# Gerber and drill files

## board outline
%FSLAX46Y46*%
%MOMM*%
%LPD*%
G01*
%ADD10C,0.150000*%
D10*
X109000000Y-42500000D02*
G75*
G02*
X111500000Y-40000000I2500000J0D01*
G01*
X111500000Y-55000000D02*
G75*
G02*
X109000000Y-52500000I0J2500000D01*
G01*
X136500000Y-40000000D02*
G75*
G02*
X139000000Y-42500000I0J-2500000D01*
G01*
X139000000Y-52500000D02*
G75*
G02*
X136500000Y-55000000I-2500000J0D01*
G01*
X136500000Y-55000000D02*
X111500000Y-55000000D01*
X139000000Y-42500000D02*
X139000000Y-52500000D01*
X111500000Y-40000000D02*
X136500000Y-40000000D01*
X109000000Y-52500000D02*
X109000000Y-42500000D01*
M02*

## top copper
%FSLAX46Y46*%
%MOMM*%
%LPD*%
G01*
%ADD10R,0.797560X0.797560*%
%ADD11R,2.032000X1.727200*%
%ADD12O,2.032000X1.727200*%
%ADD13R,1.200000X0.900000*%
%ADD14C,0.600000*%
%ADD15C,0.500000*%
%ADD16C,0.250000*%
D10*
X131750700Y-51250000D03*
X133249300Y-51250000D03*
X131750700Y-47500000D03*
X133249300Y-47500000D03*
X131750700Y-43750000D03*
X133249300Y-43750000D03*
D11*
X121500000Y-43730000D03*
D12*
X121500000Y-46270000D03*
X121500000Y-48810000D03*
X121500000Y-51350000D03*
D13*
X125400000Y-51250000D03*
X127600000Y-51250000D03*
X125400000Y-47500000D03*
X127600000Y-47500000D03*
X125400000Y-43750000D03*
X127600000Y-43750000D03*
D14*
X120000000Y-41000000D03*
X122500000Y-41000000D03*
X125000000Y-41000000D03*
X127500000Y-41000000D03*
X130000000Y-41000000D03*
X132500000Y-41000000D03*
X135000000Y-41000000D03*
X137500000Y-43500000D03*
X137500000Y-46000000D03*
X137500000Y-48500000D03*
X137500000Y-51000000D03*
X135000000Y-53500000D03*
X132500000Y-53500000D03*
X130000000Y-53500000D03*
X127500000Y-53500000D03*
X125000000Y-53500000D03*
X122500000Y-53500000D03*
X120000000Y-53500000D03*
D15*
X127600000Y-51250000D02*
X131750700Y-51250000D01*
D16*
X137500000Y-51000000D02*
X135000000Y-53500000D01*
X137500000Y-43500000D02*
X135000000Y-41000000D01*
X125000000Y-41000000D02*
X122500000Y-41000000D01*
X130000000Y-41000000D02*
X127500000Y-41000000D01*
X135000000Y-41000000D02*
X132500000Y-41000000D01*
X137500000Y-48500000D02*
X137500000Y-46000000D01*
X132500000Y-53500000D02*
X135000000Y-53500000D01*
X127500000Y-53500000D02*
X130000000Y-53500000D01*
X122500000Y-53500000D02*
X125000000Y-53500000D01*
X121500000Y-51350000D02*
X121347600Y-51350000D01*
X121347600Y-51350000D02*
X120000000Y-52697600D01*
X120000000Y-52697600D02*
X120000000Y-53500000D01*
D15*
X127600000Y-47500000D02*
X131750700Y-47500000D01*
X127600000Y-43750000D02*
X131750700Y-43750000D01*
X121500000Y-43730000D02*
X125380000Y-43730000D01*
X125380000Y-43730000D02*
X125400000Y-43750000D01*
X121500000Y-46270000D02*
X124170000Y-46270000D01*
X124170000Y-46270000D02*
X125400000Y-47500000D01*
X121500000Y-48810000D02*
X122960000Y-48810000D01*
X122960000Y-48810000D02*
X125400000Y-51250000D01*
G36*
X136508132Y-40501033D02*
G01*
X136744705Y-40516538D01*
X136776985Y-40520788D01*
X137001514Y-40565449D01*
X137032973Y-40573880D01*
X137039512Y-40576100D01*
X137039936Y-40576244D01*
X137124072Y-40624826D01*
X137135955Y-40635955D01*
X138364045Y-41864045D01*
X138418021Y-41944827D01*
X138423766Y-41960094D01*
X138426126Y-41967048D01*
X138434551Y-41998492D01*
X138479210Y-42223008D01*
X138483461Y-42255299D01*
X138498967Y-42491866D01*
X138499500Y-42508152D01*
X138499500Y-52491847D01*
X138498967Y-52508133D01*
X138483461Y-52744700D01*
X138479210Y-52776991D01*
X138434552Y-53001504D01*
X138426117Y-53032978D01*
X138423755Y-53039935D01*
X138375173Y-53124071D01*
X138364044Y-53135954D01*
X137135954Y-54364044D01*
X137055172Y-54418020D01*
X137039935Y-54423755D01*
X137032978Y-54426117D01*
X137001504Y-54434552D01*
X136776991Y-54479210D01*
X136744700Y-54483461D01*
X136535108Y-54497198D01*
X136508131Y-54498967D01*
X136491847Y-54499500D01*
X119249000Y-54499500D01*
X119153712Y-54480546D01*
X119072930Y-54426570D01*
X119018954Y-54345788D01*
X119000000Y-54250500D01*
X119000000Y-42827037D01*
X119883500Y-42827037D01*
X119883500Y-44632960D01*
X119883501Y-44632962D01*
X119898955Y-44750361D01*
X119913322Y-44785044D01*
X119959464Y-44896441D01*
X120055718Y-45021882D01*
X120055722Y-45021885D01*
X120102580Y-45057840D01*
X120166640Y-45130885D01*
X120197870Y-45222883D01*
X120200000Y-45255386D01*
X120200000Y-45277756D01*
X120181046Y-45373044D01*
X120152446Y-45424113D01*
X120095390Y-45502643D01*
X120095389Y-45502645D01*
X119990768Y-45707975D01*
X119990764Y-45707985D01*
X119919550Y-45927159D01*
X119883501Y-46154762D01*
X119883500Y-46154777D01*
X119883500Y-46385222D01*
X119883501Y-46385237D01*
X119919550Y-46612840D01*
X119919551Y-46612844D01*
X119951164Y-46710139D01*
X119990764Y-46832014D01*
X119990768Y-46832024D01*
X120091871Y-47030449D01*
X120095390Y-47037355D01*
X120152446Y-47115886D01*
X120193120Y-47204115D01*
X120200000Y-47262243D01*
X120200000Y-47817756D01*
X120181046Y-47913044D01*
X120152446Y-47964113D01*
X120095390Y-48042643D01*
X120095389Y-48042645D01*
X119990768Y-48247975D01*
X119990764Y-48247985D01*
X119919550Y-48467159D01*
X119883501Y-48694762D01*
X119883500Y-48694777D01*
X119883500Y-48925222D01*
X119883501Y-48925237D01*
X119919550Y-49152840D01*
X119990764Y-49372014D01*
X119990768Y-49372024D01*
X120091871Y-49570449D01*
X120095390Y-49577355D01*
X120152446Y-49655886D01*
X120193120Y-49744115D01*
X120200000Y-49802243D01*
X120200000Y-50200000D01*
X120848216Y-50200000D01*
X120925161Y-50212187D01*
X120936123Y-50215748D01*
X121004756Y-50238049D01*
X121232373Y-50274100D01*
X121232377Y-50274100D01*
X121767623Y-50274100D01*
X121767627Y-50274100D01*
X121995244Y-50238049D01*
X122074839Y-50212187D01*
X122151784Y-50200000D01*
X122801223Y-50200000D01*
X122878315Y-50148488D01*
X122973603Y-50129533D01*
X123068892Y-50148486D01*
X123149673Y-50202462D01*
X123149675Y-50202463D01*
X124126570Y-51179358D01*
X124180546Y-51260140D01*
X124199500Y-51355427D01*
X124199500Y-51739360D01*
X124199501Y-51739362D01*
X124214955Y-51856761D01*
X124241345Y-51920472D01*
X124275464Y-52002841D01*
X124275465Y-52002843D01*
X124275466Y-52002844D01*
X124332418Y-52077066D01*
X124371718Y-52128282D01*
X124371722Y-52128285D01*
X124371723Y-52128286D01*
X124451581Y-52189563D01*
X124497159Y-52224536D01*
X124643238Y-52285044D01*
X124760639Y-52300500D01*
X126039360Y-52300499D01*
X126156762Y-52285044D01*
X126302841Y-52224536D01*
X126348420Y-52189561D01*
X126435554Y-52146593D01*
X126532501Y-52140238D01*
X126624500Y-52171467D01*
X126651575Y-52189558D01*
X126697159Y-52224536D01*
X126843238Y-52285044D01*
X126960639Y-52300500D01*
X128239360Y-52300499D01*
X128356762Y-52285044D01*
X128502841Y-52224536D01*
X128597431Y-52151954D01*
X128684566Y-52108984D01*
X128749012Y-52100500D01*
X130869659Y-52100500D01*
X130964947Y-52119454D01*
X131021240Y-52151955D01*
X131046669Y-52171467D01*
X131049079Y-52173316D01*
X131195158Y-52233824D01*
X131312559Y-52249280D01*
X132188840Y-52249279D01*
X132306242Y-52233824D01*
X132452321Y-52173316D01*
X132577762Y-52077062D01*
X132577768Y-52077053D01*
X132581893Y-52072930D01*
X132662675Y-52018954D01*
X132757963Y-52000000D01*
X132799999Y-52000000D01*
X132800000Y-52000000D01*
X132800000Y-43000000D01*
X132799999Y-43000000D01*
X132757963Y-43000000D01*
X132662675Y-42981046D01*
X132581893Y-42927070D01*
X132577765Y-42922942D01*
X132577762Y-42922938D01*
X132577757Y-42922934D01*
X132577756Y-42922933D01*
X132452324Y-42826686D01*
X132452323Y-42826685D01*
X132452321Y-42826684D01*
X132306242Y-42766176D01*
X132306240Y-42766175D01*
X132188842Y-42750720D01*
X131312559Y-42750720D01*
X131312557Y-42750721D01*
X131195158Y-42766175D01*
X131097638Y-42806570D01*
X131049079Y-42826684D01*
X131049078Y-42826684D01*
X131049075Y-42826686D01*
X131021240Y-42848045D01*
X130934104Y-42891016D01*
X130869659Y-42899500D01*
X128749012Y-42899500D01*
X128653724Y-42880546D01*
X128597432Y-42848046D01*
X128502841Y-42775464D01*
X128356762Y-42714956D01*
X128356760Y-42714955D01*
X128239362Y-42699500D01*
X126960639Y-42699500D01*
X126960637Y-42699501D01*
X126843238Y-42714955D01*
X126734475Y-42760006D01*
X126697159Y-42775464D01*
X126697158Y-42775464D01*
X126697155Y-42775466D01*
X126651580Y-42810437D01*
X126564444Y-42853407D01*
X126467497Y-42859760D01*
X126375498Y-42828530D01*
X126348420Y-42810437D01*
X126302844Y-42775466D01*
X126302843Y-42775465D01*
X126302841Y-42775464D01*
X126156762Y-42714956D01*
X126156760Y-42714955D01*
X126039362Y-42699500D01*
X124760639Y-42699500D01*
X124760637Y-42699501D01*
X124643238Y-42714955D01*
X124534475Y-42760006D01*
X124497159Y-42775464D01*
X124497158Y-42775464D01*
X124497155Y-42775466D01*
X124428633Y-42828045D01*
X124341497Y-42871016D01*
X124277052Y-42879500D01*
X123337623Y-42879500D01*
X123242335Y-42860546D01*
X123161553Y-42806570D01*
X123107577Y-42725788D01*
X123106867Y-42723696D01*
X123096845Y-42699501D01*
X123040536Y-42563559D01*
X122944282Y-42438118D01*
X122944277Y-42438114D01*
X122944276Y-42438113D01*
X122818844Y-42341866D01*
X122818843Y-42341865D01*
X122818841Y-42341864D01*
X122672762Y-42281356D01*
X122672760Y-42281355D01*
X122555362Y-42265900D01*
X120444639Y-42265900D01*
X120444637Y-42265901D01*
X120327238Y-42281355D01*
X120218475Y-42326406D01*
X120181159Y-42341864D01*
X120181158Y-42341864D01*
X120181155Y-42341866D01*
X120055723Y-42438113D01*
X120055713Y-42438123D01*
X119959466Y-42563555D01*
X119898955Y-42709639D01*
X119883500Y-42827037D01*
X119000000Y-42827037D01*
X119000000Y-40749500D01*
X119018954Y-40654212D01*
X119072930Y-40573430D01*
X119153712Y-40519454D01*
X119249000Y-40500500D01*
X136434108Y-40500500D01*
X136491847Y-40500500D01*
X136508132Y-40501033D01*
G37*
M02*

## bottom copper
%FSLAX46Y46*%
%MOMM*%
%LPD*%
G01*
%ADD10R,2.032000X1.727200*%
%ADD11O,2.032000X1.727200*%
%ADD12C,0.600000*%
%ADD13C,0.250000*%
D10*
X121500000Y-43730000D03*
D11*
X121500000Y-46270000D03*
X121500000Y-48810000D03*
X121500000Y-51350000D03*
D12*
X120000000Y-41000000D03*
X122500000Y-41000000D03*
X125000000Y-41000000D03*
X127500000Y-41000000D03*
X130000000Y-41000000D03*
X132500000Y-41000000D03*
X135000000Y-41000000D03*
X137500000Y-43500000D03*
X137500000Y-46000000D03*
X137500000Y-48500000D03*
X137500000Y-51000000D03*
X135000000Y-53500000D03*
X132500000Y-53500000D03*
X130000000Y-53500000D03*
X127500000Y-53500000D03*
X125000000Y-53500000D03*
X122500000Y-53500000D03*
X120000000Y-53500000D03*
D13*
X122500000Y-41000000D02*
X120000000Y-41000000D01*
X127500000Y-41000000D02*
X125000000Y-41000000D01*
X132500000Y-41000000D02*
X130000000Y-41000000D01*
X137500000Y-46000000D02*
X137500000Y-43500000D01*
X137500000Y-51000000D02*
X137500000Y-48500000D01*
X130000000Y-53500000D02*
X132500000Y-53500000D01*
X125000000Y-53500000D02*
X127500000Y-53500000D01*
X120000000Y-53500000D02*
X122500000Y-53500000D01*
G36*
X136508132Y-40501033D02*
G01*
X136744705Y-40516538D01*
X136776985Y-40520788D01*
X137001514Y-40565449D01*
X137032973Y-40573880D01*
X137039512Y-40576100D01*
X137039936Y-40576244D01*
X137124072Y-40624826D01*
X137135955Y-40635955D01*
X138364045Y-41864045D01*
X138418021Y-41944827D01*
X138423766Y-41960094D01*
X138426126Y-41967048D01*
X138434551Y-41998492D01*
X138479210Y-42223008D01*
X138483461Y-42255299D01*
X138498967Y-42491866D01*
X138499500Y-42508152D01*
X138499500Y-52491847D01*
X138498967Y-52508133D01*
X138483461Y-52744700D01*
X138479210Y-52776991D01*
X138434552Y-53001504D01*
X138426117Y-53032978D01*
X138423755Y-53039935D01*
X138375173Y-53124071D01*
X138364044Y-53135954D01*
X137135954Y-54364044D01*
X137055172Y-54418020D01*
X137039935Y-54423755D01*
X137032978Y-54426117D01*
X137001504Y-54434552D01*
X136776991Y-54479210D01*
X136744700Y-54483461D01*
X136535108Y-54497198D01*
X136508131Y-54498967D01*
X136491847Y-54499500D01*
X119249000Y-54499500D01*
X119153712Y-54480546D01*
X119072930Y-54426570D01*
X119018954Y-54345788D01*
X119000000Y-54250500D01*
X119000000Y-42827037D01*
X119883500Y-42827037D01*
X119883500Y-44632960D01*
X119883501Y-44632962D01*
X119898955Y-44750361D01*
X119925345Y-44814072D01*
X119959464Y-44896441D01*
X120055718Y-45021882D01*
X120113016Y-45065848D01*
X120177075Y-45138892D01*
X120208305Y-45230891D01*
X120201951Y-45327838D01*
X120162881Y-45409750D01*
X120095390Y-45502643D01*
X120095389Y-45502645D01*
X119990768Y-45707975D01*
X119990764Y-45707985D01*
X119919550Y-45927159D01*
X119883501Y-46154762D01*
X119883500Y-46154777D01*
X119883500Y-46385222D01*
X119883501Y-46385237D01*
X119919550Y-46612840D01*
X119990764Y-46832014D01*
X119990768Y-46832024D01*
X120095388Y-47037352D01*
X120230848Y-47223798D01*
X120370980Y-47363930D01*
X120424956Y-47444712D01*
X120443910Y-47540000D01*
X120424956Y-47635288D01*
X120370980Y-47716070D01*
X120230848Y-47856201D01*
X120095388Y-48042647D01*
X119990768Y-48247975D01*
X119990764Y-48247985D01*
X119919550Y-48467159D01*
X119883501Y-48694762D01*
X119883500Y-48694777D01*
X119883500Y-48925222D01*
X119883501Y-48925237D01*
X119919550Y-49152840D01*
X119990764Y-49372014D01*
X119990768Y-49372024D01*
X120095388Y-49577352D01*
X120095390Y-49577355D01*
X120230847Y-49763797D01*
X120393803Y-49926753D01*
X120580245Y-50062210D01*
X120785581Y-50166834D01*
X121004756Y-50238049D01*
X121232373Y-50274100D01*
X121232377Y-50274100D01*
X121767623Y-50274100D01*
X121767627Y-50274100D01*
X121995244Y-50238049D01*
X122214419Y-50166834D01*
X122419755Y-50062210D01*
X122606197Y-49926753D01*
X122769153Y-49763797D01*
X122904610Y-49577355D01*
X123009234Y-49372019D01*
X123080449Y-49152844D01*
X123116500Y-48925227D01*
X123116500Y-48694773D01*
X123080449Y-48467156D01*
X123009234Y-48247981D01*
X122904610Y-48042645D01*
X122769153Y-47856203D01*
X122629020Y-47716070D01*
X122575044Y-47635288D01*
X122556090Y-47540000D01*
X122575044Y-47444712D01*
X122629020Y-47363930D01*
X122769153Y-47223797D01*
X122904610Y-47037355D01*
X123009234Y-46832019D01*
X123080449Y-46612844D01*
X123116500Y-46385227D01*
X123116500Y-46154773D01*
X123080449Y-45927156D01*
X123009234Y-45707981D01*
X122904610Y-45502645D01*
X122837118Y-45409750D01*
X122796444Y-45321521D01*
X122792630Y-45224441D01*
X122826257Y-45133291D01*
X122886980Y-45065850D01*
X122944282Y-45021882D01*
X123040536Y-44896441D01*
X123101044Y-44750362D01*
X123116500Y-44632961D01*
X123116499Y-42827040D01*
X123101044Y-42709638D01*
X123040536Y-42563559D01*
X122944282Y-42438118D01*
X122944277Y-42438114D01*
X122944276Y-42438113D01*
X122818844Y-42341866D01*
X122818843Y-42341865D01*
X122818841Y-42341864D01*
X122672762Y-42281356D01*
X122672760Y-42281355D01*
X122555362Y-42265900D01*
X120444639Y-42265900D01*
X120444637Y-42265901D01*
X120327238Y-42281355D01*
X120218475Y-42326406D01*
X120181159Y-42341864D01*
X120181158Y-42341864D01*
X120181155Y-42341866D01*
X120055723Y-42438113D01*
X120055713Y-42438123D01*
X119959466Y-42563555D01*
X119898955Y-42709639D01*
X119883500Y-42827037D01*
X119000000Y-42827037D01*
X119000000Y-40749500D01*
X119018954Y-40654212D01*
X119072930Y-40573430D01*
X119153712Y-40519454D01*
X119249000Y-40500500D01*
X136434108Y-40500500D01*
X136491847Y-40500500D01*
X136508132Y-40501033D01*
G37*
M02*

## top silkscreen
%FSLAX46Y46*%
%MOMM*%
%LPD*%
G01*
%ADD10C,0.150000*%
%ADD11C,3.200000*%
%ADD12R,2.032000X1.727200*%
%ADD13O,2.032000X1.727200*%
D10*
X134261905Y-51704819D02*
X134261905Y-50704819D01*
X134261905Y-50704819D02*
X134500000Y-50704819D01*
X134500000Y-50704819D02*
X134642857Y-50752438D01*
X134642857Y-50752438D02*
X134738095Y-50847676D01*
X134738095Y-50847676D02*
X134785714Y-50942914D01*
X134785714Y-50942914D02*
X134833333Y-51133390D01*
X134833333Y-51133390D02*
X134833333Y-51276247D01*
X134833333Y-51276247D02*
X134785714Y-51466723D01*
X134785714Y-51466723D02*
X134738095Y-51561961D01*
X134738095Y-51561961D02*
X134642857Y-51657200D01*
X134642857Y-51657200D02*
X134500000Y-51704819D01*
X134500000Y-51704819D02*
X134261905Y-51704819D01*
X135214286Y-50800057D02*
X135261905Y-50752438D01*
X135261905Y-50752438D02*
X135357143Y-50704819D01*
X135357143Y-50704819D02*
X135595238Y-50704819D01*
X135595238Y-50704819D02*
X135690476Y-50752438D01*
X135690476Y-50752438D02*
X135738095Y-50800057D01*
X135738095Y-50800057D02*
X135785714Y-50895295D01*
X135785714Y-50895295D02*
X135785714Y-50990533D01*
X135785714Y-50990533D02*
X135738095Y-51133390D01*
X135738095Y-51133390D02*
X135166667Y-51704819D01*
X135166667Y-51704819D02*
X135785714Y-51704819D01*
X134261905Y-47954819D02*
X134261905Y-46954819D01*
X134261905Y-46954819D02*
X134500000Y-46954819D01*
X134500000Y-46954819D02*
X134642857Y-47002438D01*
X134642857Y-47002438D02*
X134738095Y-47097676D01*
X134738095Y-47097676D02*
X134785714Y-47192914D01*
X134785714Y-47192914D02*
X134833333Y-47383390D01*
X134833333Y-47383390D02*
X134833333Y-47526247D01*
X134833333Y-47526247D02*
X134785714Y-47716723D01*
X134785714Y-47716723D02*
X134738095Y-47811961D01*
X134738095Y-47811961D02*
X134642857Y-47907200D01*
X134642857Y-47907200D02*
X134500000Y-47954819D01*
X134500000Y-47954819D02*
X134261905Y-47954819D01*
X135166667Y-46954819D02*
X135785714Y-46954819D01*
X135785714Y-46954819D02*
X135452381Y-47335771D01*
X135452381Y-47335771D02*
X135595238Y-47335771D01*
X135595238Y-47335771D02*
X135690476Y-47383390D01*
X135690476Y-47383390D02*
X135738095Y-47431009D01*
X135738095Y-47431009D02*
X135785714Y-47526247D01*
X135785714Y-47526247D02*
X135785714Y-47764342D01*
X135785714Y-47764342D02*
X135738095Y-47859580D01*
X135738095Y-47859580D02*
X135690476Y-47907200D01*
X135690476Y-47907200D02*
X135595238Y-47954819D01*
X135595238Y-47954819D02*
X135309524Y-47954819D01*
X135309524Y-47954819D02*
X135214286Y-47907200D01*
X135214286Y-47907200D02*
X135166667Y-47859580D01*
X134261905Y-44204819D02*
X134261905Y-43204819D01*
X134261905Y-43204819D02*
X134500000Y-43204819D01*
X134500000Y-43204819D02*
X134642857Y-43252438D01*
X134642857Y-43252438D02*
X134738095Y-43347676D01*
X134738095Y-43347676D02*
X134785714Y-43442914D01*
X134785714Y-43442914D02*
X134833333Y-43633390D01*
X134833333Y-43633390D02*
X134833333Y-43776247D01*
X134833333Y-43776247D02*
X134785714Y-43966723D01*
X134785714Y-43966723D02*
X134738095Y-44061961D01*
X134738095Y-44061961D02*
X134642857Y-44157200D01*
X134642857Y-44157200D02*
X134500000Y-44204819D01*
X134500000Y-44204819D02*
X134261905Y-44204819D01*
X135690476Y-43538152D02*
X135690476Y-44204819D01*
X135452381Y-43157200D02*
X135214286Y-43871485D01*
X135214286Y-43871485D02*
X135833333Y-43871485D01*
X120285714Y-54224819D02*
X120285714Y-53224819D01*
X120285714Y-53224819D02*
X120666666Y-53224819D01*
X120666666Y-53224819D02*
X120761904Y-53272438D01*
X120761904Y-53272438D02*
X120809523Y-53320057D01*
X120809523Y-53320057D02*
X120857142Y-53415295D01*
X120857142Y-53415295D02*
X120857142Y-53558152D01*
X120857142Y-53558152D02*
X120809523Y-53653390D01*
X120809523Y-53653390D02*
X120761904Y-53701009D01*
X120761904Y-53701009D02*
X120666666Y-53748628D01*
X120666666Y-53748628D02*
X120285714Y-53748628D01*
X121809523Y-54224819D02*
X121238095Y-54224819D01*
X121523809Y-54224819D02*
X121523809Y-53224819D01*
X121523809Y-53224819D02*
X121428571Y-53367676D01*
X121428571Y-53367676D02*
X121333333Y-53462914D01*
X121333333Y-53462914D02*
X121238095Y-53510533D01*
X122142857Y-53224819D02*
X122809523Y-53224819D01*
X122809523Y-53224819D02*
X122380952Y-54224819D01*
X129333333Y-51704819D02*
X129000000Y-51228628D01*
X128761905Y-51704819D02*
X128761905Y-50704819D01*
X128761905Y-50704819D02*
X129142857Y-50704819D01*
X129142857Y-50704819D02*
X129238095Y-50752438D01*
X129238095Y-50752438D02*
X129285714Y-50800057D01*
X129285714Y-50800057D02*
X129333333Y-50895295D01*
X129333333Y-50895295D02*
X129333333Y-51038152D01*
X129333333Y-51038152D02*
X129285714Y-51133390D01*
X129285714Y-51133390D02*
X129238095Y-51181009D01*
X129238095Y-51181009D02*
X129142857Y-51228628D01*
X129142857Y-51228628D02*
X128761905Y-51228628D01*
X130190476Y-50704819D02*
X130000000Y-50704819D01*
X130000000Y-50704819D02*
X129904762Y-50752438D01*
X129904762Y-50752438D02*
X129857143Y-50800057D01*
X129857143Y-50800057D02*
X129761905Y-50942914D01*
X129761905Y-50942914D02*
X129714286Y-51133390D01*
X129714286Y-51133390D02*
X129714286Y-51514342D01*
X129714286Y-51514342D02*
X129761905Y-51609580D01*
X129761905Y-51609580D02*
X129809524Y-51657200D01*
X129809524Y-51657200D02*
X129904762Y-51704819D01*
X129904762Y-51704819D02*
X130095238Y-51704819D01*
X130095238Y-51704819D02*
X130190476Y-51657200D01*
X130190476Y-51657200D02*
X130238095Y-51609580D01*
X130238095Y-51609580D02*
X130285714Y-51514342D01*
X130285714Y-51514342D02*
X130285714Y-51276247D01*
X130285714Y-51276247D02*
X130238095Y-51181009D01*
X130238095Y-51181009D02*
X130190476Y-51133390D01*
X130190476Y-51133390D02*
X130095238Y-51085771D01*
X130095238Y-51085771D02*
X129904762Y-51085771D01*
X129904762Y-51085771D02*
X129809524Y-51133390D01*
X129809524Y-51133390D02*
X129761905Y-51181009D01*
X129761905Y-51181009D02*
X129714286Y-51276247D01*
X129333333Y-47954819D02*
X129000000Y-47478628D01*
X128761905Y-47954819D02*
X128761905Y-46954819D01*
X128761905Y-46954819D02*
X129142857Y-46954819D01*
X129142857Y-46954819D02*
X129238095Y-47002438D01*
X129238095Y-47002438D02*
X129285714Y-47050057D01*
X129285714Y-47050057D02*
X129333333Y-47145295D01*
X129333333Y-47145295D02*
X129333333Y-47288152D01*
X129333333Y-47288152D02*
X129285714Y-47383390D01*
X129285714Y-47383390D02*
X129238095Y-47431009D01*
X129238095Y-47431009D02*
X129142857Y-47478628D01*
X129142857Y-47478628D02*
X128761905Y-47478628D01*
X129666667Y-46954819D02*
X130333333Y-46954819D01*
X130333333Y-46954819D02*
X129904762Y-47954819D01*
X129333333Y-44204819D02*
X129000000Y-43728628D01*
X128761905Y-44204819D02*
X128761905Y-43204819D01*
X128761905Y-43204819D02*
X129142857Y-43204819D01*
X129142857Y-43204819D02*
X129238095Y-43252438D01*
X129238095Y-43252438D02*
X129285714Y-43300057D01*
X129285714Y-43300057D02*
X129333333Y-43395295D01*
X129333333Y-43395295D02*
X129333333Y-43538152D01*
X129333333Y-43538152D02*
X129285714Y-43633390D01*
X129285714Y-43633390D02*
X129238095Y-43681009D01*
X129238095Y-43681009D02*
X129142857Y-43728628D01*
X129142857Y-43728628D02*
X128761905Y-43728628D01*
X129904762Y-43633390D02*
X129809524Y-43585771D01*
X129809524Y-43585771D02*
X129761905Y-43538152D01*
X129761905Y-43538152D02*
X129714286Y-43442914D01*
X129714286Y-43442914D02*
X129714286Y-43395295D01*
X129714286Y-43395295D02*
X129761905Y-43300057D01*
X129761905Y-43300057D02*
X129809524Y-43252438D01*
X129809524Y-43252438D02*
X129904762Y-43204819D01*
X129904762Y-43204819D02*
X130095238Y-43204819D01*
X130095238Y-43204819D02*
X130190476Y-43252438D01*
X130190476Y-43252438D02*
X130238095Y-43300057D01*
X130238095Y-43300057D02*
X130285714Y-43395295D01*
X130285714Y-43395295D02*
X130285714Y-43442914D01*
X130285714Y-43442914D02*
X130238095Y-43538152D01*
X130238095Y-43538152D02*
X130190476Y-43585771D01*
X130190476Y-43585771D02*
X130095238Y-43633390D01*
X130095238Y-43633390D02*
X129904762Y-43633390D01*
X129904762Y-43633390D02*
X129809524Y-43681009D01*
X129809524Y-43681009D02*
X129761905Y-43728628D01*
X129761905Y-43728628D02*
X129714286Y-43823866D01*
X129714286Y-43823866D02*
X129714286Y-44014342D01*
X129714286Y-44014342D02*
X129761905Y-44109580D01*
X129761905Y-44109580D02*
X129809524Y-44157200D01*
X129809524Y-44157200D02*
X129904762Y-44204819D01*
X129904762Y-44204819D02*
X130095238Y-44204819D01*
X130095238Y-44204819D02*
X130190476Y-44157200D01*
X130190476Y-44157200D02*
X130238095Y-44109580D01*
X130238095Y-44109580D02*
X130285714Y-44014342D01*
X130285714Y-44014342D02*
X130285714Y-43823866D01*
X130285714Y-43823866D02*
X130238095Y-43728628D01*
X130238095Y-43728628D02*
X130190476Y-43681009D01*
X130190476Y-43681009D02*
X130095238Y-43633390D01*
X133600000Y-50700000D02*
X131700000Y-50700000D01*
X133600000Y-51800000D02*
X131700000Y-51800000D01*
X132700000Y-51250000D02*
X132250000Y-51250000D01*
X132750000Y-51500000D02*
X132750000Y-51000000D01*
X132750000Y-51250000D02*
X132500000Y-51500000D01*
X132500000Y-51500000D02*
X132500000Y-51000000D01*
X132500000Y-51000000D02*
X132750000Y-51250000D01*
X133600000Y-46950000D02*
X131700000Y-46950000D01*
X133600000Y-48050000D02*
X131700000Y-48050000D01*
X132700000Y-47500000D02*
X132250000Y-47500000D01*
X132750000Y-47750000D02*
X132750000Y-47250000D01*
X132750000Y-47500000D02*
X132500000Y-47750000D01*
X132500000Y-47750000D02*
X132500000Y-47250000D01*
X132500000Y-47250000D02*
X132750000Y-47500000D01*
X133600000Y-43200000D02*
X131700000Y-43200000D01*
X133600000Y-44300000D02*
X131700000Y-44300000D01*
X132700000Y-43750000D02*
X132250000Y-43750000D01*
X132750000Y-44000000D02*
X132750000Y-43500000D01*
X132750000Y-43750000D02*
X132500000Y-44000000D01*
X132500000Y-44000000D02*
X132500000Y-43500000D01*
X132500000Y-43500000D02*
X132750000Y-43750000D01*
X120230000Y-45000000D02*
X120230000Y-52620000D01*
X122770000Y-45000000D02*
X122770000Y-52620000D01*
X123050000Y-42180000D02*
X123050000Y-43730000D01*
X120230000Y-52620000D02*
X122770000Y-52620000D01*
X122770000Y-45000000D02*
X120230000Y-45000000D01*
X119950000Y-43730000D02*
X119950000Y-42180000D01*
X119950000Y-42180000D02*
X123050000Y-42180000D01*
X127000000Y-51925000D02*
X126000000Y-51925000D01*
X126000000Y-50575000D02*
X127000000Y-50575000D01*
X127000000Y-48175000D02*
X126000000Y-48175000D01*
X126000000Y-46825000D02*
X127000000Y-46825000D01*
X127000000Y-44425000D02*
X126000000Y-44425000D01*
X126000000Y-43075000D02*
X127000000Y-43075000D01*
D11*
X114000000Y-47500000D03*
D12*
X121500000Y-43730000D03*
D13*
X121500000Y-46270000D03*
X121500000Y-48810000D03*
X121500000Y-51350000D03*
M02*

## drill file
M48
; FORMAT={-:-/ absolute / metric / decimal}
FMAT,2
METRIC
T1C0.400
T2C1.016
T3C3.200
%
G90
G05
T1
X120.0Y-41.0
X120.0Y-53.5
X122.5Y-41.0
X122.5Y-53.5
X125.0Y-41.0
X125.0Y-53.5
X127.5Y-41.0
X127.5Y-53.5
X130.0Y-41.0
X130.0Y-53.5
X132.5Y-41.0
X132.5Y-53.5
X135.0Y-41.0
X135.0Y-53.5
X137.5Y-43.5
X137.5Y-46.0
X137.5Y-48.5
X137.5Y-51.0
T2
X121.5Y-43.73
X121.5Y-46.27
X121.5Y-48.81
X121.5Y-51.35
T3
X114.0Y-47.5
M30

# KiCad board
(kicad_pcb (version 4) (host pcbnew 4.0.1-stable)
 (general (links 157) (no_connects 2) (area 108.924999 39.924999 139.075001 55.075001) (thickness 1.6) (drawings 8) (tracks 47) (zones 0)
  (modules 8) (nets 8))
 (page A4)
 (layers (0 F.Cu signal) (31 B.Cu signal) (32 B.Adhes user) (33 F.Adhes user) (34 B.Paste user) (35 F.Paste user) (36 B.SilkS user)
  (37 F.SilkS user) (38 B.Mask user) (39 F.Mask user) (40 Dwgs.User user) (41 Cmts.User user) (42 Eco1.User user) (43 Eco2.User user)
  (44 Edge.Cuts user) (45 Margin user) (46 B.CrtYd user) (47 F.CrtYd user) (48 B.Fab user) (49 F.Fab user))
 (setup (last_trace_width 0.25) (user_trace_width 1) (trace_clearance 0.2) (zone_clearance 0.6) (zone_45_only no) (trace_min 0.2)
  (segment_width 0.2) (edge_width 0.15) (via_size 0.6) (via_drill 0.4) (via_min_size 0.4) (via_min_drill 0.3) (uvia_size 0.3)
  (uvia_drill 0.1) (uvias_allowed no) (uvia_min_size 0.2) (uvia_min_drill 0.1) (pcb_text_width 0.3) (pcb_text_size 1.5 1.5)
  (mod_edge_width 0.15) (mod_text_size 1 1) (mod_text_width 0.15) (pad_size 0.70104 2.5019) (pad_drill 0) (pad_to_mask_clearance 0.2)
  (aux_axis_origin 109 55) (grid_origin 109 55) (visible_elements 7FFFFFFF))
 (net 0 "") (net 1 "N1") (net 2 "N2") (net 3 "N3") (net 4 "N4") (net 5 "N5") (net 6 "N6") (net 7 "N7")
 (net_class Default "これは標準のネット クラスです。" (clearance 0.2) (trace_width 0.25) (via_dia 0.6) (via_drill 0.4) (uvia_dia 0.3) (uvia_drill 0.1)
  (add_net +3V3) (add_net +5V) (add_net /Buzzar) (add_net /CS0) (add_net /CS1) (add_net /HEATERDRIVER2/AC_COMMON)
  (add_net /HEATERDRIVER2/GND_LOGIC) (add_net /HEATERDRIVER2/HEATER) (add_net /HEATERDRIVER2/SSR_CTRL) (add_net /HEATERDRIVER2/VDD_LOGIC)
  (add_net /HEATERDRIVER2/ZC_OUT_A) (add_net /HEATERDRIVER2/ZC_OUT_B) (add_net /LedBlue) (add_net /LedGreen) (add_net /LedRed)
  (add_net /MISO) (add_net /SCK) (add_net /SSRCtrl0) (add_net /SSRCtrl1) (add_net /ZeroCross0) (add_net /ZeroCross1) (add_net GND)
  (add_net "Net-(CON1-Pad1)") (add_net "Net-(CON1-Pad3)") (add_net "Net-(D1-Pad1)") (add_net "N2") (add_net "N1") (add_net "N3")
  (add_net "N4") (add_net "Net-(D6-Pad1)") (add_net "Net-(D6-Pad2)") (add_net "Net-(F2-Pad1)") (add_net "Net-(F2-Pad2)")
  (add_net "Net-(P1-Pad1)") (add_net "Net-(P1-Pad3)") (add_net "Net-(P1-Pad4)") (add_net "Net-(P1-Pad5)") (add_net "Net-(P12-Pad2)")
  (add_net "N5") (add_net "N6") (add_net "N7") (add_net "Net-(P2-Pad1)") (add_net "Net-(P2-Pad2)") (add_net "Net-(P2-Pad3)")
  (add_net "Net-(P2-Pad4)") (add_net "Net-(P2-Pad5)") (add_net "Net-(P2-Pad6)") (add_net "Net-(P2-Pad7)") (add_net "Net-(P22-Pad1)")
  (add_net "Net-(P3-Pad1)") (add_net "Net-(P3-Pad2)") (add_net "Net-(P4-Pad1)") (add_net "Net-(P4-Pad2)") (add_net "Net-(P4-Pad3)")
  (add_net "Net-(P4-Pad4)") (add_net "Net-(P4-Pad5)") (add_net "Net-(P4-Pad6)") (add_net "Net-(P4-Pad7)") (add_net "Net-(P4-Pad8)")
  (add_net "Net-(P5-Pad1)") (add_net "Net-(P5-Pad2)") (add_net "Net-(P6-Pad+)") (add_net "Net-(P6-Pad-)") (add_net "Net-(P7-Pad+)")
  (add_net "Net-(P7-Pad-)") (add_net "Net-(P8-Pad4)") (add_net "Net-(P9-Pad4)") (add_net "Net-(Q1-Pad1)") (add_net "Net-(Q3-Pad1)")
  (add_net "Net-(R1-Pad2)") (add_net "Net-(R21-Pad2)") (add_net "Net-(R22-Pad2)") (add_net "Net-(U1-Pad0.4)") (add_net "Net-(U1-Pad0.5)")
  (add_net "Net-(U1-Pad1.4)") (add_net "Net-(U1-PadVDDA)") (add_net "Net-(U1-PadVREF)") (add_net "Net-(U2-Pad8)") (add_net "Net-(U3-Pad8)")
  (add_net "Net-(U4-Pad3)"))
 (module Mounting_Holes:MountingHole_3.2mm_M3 (layer F.Cu) (at 114 47.5 90)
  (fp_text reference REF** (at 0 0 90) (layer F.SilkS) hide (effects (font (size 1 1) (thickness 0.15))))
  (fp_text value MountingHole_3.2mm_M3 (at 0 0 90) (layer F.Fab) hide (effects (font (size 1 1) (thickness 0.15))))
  (pad 1 np_thru_hole circle (at 0 0 90) (size 3.2 3.2) (drill 3.2) (layers *.Cu *.Mask F.SilkS)))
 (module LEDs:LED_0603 (layer F.Cu) (at 132.5 51.25 180)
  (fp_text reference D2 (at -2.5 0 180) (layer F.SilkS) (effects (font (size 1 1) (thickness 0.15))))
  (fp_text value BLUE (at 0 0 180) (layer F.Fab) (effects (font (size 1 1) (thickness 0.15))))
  (fp_line (start -1.1 0.55) (end 0.8 0.55) (layer F.SilkS) (width 0.15))
  (fp_line (start -1.1 -0.55) (end 0.8 -0.55) (layer F.SilkS) (width 0.15))
  (fp_line (start -0.2 0) (end 0.25 0) (layer F.SilkS) (width 0.15))
  (fp_line (start -0.25 -0.25) (end -0.25 0.25) (layer F.SilkS) (width 0.15))
  (fp_line (start -0.25 0) (end 0 -0.25) (layer F.SilkS) (width 0.15))
  (fp_line (start 0 -0.25) (end 0 0.25) (layer F.SilkS) (width 0.15))
  (fp_line (start 0 0.25) (end -0.25 0) (layer F.SilkS) (width 0.15))
  (pad 2 smd rect (at 0.7493 0) (size 0.79756 0.79756) (layers F.Cu F.Paste F.Mask) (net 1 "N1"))
  (pad 1 smd rect (at -0.7493 0) (size 0.79756 0.79756) (layers F.Cu F.Paste F.Mask) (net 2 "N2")))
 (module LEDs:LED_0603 (layer F.Cu) (at 132.5 47.5 180)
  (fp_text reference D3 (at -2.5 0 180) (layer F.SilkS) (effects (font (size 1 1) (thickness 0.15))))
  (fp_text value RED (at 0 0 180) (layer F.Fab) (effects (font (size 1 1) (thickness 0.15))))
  (fp_line (start -1.1 0.55) (end 0.8 0.55) (layer F.SilkS) (width 0.15))
  (fp_line (start -1.1 -0.55) (end 0.8 -0.55) (layer F.SilkS) (width 0.15))
  (fp_line (start -0.2 0) (end 0.25 0) (layer F.SilkS) (width 0.15))
  (fp_line (start -0.25 -0.25) (end -0.25 0.25) (layer F.SilkS) (width 0.15))
  (fp_line (start -0.25 0) (end 0 -0.25) (layer F.SilkS) (width 0.15))
  (fp_line (start 0 -0.25) (end 0 0.25) (layer F.SilkS) (width 0.15))
  (fp_line (start 0 0.25) (end -0.25 0) (layer F.SilkS) (width 0.15))
  (pad 2 smd rect (at 0.7493 0) (size 0.79756 0.79756) (layers F.Cu F.Paste F.Mask) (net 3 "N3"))
  (pad 1 smd rect (at -0.7493 0) (size 0.79756 0.79756) (layers F.Cu F.Paste F.Mask) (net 2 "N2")))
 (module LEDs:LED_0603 (layer F.Cu) (at 132.5 43.75 180)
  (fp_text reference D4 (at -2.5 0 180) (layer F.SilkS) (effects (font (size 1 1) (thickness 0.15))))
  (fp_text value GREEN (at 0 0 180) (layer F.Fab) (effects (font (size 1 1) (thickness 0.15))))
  (fp_line (start -1.1 0.55) (end 0.8 0.55) (layer F.SilkS) (width 0.15))
  (fp_line (start -1.1 -0.55) (end 0.8 -0.55) (layer F.SilkS) (width 0.15))
  (fp_line (start -0.2 0) (end 0.25 0) (layer F.SilkS) (width 0.15))
  (fp_line (start -0.25 -0.25) (end -0.25 0.25) (layer F.SilkS) (width 0.15))
  (fp_line (start -0.25 0) (end 0 -0.25) (layer F.SilkS) (width 0.15))
  (fp_line (start 0 -0.25) (end 0 0.25) (layer F.SilkS) (width 0.15))
  (fp_line (start 0 0.25) (end -0.25 0) (layer F.SilkS) (width 0.15))
  (pad 2 smd rect (at 0.7493 0) (size 0.79756 0.79756) (layers F.Cu F.Paste F.Mask) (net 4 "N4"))
  (pad 1 smd rect (at -0.7493 0) (size 0.79756 0.79756) (layers F.Cu F.Paste F.Mask) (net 2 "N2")))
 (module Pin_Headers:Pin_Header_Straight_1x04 (layer F.Cu) (at 121.5 43.73)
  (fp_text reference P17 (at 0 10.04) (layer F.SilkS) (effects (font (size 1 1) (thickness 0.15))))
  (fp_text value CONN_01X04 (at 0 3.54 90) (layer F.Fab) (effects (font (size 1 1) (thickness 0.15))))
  (fp_line (start -1.27 1.27) (end -1.27 8.89) (layer F.SilkS) (width 0.15))
  (fp_line (start 1.27 1.27) (end 1.27 8.89) (layer F.SilkS) (width 0.15))
  (fp_line (start 1.55 -1.55) (end 1.55 0) (layer F.SilkS) (width 0.15))
  (fp_line (start -1.27 8.89) (end 1.27 8.89) (layer F.SilkS) (width 0.15))
  (fp_line (start 1.27 1.27) (end -1.27 1.27) (layer F.SilkS) (width 0.15))
  (fp_line (start -1.55 0) (end -1.55 -1.55) (layer F.SilkS) (width 0.15))
  (fp_line (start -1.55 -1.55) (end 1.55 -1.55) (layer F.SilkS) (width 0.15))
  (pad 1 thru_hole rect (at 0 0) (size 2.032 1.7272) (drill 1.016) (layers *.Cu *.Mask F.SilkS) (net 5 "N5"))
  (pad 2 thru_hole oval (at 0 2.54) (size 2.032 1.7272) (drill 1.016) (layers *.Cu *.Mask F.SilkS) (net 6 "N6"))
  (pad 3 thru_hole oval (at 0 5.08) (size 2.032 1.7272) (drill 1.016) (layers *.Cu *.Mask F.SilkS) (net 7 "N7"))
  (pad 4 thru_hole oval (at 0 7.62) (size 2.032 1.7272) (drill 1.016) (layers *.Cu *.Mask F.SilkS) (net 2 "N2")))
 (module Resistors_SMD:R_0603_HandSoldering (layer F.Cu) (at 126.5 51.25)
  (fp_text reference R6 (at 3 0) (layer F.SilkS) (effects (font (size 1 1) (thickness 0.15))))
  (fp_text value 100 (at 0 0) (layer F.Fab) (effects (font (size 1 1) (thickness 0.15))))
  (fp_line (start 0.5 0.675) (end -0.5 0.675) (layer F.SilkS) (width 0.15))
  (fp_line (start -0.5 -0.675) (end 0.5 -0.675) (layer F.SilkS) (width 0.15))
  (pad 1 smd rect (at -1.1 0) (size 1.2 0.9) (layers F.Cu F.Paste F.Mask) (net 7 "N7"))
  (pad 2 smd rect (at 1.1 0) (size 1.2 0.9) (layers F.Cu F.Paste F.Mask) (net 1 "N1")))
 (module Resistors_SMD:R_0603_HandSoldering (layer F.Cu) (at 126.5 47.5)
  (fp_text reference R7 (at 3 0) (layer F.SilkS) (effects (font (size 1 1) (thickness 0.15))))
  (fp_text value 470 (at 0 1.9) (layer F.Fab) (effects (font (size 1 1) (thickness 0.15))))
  (fp_line (start 0.5 0.675) (end -0.5 0.675) (layer F.SilkS) (width 0.15))
  (fp_line (start -0.5 -0.675) (end 0.5 -0.675) (layer F.SilkS) (width 0.15))
  (pad 1 smd rect (at -1.1 0) (size 1.2 0.9) (layers F.Cu F.Paste F.Mask) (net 6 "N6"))
  (pad 2 smd rect (at 1.1 0) (size 1.2 0.9) (layers F.Cu F.Paste F.Mask) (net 3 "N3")))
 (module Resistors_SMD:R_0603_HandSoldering (layer F.Cu) (at 126.5 43.75)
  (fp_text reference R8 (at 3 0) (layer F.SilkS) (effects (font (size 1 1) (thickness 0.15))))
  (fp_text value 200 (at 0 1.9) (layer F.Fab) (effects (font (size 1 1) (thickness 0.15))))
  (fp_line (start 0.5 0.675) (end -0.5 0.675) (layer F.SilkS) (width 0.15))
  (fp_line (start -0.5 -0.675) (end 0.5 -0.675) (layer F.SilkS) (width 0.15))
  (pad 1 smd rect (at -1.1 0) (size 1.2 0.9) (layers F.Cu F.Paste F.Mask) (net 5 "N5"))
  (pad 2 smd rect (at 1.1 0) (size 1.2 0.9) (layers F.Cu F.Paste F.Mask) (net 4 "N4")))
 (gr_arc (start 111.5 42.5) (end 109 42.5) (angle 90) (layer Edge.Cuts) (width 0.15))
 (gr_arc (start 111.5 52.5) (end 111.5 55) (angle 90) (layer Edge.Cuts) (width 0.15))
 (gr_arc (start 136.5 42.5) (end 136.5 40) (angle 90) (layer Edge.Cuts) (width 0.15))
 (gr_arc (start 136.5 52.5) (end 139 52.5) (angle 90) (layer Edge.Cuts) (width 0.15))
 (gr_line (start 136.5 55) (end 111.5 55) (layer Edge.Cuts) (width 0.15))
 (gr_line (start 139 42.5) (end 139 52.5) (layer Edge.Cuts) (width 0.15))
 (gr_line (start 111.5 40) (end 136.5 40) (layer Edge.Cuts) (width 0.15))
 (gr_line (start 109 52.5) (end 109 42.5) (layer Edge.Cuts) (width 0.15))
 (segment (start 127.6 51.25) (end 131.7507 51.25) (width 0.5) (layer F.Cu) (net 1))
 (segment (start 137.5 51) (end 135 53.5) (width 0.25) (layer F.Cu) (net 2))
 (segment (start 137.5 43.5) (end 135 41) (width 0.25) (layer F.Cu) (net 2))
 (segment (start 122.5 41) (end 120 41) (width 0.25) (layer B.Cu) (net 2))
 (via (at 120 41) (size 0.6) (drill 0.4) (layers F.Cu B.Cu) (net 2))
 (segment (start 125 41) (end 122.5 41) (width 0.25) (layer F.Cu) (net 2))
 (via (at 122.5 41) (size 0.6) (drill 0.4) (layers F.Cu B.Cu) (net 2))
 (segment (start 127.5 41) (end 125 41) (width 0.25) (layer B.Cu) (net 2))
 (via (at 125 41) (size 0.6) (drill 0.4) (layers F.Cu B.Cu) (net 2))
 (segment (start 130 41) (end 127.5 41) (width 0.25) (layer F.Cu) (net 2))
 (via (at 127.5 41) (size 0.6) (drill 0.4) (layers F.Cu B.Cu) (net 2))
 (segment (start 132.5 41) (end 130 41) (width 0.25) (layer B.Cu) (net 2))
 (via (at 130 41) (size 0.6) (drill 0.4) (layers F.Cu B.Cu) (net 2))
 (segment (start 135 41) (end 132.5 41) (width 0.25) (layer F.Cu) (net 2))
 (via (at 132.5 41) (size 0.6) (drill 0.4) (layers F.Cu B.Cu) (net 2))
 (via (at 135 41) (size 0.6) (drill 0.4) (layers F.Cu B.Cu) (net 2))
 (segment (start 137.5 46) (end 137.5 43.5) (width 0.25) (layer B.Cu) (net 2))
 (via (at 137.5 43.5) (size 0.6) (drill 0.4) (layers F.Cu B.Cu) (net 2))
 (segment (start 137.5 48.5) (end 137.5 46) (width 0.25) (layer F.Cu) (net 2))
 (via (at 137.5 46) (size 0.6) (drill 0.4) (layers F.Cu B.Cu) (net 2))
 (segment (start 137.5 51) (end 137.5 48.5) (width 0.25) (layer B.Cu) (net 2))
 (via (at 137.5 48.5) (size 0.6) (drill 0.4) (layers F.Cu B.Cu) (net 2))
 (via (at 137.5 51) (size 0.6) (drill 0.4) (layers F.Cu B.Cu) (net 2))
 (segment (start 132.5 53.5) (end 135 53.5) (width 0.25) (layer F.Cu) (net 2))
 (via (at 135 53.5) (size 0.6) (drill 0.4) (layers F.Cu B.Cu) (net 2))
 (segment (start 130 53.5) (end 132.5 53.5) (width 0.25) (layer B.Cu) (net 2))
 (via (at 132.5 53.5) (size 0.6) (drill 0.4) (layers F.Cu B.Cu) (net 2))
 (segment (start 127.5 53.5) (end 130 53.5) (width 0.25) (layer F.Cu) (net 2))
 (via (at 130 53.5) (size 0.6) (drill 0.4) (layers F.Cu B.Cu) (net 2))
 (segment (start 125 53.5) (end 127.5 53.5) (width 0.25) (layer B.Cu) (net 2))
 (via (at 127.5 53.5) (size 0.6) (drill 0.4) (layers F.Cu B.Cu) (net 2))
 (segment (start 122.5 53.5) (end 125 53.5) (width 0.25) (layer F.Cu) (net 2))
 (via (at 125 53.5) (size 0.6) (drill 0.4) (layers F.Cu B.Cu) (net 2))
 (segment (start 120 53.5) (end 122.5 53.5) (width 0.25) (layer B.Cu) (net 2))
 (via (at 122.5 53.5) (size 0.6) (drill 0.4) (layers F.Cu B.Cu) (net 2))
 (segment (start 121.5 51.35) (end 121.3476 51.35) (width 0.25) (layer F.Cu) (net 2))
 (segment (start 121.3476 51.35) (end 120 52.6976) (width 0.25) (layer F.Cu) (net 2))
 (segment (start 120 52.6976) (end 120 53.5) (width 0.25) (layer F.Cu) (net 2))
 (via (at 120 53.5) (size 0.6) (drill 0.4) (layers F.Cu B.Cu) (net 2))
 (segment (start 127.6 47.5) (end 131.7507 47.5) (width 0.5) (layer F.Cu) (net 3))
 (segment (start 127.6 43.75) (end 131.7507 43.75) (width 0.5) (layer F.Cu) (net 4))
 (segment (start 121.5 43.73) (end 125.38 43.73) (width 0.5) (layer F.Cu) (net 5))
 (segment (start 125.38 43.73) (end 125.4 43.75) (width 0.5) (layer F.Cu) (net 5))
 (segment (start 121.5 46.27) (end 124.17 46.27) (width 0.5) (layer F.Cu) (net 6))
 (segment (start 124.17 46.27) (end 125.4 47.5) (width 0.5) (layer F.Cu) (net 6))
 (segment (start 121.5 48.81) (end 122.96 48.81) (width 0.5) (layer F.Cu) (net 7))
 (segment (start 122.96 48.81) (end 125.4 51.25) (width 0.5) (layer F.Cu) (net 7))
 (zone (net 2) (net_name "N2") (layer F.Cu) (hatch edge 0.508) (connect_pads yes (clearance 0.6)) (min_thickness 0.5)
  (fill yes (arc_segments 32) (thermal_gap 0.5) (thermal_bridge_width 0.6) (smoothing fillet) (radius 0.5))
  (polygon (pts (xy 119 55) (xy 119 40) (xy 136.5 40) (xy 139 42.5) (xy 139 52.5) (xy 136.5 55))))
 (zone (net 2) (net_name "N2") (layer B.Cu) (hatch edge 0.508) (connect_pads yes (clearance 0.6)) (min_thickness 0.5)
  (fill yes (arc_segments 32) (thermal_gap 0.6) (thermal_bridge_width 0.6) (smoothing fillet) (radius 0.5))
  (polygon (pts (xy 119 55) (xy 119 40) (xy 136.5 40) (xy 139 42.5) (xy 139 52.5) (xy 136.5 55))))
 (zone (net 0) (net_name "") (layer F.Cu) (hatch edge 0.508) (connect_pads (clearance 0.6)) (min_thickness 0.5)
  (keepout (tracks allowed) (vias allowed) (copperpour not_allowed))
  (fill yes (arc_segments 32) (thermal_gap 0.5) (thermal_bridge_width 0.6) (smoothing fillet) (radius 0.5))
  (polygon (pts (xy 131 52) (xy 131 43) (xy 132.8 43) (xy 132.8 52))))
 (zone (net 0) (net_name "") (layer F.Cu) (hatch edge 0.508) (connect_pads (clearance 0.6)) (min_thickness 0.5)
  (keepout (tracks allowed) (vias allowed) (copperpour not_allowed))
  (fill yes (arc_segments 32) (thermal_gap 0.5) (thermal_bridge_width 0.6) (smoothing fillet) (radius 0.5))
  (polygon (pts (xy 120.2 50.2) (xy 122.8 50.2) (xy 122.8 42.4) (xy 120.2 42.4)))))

